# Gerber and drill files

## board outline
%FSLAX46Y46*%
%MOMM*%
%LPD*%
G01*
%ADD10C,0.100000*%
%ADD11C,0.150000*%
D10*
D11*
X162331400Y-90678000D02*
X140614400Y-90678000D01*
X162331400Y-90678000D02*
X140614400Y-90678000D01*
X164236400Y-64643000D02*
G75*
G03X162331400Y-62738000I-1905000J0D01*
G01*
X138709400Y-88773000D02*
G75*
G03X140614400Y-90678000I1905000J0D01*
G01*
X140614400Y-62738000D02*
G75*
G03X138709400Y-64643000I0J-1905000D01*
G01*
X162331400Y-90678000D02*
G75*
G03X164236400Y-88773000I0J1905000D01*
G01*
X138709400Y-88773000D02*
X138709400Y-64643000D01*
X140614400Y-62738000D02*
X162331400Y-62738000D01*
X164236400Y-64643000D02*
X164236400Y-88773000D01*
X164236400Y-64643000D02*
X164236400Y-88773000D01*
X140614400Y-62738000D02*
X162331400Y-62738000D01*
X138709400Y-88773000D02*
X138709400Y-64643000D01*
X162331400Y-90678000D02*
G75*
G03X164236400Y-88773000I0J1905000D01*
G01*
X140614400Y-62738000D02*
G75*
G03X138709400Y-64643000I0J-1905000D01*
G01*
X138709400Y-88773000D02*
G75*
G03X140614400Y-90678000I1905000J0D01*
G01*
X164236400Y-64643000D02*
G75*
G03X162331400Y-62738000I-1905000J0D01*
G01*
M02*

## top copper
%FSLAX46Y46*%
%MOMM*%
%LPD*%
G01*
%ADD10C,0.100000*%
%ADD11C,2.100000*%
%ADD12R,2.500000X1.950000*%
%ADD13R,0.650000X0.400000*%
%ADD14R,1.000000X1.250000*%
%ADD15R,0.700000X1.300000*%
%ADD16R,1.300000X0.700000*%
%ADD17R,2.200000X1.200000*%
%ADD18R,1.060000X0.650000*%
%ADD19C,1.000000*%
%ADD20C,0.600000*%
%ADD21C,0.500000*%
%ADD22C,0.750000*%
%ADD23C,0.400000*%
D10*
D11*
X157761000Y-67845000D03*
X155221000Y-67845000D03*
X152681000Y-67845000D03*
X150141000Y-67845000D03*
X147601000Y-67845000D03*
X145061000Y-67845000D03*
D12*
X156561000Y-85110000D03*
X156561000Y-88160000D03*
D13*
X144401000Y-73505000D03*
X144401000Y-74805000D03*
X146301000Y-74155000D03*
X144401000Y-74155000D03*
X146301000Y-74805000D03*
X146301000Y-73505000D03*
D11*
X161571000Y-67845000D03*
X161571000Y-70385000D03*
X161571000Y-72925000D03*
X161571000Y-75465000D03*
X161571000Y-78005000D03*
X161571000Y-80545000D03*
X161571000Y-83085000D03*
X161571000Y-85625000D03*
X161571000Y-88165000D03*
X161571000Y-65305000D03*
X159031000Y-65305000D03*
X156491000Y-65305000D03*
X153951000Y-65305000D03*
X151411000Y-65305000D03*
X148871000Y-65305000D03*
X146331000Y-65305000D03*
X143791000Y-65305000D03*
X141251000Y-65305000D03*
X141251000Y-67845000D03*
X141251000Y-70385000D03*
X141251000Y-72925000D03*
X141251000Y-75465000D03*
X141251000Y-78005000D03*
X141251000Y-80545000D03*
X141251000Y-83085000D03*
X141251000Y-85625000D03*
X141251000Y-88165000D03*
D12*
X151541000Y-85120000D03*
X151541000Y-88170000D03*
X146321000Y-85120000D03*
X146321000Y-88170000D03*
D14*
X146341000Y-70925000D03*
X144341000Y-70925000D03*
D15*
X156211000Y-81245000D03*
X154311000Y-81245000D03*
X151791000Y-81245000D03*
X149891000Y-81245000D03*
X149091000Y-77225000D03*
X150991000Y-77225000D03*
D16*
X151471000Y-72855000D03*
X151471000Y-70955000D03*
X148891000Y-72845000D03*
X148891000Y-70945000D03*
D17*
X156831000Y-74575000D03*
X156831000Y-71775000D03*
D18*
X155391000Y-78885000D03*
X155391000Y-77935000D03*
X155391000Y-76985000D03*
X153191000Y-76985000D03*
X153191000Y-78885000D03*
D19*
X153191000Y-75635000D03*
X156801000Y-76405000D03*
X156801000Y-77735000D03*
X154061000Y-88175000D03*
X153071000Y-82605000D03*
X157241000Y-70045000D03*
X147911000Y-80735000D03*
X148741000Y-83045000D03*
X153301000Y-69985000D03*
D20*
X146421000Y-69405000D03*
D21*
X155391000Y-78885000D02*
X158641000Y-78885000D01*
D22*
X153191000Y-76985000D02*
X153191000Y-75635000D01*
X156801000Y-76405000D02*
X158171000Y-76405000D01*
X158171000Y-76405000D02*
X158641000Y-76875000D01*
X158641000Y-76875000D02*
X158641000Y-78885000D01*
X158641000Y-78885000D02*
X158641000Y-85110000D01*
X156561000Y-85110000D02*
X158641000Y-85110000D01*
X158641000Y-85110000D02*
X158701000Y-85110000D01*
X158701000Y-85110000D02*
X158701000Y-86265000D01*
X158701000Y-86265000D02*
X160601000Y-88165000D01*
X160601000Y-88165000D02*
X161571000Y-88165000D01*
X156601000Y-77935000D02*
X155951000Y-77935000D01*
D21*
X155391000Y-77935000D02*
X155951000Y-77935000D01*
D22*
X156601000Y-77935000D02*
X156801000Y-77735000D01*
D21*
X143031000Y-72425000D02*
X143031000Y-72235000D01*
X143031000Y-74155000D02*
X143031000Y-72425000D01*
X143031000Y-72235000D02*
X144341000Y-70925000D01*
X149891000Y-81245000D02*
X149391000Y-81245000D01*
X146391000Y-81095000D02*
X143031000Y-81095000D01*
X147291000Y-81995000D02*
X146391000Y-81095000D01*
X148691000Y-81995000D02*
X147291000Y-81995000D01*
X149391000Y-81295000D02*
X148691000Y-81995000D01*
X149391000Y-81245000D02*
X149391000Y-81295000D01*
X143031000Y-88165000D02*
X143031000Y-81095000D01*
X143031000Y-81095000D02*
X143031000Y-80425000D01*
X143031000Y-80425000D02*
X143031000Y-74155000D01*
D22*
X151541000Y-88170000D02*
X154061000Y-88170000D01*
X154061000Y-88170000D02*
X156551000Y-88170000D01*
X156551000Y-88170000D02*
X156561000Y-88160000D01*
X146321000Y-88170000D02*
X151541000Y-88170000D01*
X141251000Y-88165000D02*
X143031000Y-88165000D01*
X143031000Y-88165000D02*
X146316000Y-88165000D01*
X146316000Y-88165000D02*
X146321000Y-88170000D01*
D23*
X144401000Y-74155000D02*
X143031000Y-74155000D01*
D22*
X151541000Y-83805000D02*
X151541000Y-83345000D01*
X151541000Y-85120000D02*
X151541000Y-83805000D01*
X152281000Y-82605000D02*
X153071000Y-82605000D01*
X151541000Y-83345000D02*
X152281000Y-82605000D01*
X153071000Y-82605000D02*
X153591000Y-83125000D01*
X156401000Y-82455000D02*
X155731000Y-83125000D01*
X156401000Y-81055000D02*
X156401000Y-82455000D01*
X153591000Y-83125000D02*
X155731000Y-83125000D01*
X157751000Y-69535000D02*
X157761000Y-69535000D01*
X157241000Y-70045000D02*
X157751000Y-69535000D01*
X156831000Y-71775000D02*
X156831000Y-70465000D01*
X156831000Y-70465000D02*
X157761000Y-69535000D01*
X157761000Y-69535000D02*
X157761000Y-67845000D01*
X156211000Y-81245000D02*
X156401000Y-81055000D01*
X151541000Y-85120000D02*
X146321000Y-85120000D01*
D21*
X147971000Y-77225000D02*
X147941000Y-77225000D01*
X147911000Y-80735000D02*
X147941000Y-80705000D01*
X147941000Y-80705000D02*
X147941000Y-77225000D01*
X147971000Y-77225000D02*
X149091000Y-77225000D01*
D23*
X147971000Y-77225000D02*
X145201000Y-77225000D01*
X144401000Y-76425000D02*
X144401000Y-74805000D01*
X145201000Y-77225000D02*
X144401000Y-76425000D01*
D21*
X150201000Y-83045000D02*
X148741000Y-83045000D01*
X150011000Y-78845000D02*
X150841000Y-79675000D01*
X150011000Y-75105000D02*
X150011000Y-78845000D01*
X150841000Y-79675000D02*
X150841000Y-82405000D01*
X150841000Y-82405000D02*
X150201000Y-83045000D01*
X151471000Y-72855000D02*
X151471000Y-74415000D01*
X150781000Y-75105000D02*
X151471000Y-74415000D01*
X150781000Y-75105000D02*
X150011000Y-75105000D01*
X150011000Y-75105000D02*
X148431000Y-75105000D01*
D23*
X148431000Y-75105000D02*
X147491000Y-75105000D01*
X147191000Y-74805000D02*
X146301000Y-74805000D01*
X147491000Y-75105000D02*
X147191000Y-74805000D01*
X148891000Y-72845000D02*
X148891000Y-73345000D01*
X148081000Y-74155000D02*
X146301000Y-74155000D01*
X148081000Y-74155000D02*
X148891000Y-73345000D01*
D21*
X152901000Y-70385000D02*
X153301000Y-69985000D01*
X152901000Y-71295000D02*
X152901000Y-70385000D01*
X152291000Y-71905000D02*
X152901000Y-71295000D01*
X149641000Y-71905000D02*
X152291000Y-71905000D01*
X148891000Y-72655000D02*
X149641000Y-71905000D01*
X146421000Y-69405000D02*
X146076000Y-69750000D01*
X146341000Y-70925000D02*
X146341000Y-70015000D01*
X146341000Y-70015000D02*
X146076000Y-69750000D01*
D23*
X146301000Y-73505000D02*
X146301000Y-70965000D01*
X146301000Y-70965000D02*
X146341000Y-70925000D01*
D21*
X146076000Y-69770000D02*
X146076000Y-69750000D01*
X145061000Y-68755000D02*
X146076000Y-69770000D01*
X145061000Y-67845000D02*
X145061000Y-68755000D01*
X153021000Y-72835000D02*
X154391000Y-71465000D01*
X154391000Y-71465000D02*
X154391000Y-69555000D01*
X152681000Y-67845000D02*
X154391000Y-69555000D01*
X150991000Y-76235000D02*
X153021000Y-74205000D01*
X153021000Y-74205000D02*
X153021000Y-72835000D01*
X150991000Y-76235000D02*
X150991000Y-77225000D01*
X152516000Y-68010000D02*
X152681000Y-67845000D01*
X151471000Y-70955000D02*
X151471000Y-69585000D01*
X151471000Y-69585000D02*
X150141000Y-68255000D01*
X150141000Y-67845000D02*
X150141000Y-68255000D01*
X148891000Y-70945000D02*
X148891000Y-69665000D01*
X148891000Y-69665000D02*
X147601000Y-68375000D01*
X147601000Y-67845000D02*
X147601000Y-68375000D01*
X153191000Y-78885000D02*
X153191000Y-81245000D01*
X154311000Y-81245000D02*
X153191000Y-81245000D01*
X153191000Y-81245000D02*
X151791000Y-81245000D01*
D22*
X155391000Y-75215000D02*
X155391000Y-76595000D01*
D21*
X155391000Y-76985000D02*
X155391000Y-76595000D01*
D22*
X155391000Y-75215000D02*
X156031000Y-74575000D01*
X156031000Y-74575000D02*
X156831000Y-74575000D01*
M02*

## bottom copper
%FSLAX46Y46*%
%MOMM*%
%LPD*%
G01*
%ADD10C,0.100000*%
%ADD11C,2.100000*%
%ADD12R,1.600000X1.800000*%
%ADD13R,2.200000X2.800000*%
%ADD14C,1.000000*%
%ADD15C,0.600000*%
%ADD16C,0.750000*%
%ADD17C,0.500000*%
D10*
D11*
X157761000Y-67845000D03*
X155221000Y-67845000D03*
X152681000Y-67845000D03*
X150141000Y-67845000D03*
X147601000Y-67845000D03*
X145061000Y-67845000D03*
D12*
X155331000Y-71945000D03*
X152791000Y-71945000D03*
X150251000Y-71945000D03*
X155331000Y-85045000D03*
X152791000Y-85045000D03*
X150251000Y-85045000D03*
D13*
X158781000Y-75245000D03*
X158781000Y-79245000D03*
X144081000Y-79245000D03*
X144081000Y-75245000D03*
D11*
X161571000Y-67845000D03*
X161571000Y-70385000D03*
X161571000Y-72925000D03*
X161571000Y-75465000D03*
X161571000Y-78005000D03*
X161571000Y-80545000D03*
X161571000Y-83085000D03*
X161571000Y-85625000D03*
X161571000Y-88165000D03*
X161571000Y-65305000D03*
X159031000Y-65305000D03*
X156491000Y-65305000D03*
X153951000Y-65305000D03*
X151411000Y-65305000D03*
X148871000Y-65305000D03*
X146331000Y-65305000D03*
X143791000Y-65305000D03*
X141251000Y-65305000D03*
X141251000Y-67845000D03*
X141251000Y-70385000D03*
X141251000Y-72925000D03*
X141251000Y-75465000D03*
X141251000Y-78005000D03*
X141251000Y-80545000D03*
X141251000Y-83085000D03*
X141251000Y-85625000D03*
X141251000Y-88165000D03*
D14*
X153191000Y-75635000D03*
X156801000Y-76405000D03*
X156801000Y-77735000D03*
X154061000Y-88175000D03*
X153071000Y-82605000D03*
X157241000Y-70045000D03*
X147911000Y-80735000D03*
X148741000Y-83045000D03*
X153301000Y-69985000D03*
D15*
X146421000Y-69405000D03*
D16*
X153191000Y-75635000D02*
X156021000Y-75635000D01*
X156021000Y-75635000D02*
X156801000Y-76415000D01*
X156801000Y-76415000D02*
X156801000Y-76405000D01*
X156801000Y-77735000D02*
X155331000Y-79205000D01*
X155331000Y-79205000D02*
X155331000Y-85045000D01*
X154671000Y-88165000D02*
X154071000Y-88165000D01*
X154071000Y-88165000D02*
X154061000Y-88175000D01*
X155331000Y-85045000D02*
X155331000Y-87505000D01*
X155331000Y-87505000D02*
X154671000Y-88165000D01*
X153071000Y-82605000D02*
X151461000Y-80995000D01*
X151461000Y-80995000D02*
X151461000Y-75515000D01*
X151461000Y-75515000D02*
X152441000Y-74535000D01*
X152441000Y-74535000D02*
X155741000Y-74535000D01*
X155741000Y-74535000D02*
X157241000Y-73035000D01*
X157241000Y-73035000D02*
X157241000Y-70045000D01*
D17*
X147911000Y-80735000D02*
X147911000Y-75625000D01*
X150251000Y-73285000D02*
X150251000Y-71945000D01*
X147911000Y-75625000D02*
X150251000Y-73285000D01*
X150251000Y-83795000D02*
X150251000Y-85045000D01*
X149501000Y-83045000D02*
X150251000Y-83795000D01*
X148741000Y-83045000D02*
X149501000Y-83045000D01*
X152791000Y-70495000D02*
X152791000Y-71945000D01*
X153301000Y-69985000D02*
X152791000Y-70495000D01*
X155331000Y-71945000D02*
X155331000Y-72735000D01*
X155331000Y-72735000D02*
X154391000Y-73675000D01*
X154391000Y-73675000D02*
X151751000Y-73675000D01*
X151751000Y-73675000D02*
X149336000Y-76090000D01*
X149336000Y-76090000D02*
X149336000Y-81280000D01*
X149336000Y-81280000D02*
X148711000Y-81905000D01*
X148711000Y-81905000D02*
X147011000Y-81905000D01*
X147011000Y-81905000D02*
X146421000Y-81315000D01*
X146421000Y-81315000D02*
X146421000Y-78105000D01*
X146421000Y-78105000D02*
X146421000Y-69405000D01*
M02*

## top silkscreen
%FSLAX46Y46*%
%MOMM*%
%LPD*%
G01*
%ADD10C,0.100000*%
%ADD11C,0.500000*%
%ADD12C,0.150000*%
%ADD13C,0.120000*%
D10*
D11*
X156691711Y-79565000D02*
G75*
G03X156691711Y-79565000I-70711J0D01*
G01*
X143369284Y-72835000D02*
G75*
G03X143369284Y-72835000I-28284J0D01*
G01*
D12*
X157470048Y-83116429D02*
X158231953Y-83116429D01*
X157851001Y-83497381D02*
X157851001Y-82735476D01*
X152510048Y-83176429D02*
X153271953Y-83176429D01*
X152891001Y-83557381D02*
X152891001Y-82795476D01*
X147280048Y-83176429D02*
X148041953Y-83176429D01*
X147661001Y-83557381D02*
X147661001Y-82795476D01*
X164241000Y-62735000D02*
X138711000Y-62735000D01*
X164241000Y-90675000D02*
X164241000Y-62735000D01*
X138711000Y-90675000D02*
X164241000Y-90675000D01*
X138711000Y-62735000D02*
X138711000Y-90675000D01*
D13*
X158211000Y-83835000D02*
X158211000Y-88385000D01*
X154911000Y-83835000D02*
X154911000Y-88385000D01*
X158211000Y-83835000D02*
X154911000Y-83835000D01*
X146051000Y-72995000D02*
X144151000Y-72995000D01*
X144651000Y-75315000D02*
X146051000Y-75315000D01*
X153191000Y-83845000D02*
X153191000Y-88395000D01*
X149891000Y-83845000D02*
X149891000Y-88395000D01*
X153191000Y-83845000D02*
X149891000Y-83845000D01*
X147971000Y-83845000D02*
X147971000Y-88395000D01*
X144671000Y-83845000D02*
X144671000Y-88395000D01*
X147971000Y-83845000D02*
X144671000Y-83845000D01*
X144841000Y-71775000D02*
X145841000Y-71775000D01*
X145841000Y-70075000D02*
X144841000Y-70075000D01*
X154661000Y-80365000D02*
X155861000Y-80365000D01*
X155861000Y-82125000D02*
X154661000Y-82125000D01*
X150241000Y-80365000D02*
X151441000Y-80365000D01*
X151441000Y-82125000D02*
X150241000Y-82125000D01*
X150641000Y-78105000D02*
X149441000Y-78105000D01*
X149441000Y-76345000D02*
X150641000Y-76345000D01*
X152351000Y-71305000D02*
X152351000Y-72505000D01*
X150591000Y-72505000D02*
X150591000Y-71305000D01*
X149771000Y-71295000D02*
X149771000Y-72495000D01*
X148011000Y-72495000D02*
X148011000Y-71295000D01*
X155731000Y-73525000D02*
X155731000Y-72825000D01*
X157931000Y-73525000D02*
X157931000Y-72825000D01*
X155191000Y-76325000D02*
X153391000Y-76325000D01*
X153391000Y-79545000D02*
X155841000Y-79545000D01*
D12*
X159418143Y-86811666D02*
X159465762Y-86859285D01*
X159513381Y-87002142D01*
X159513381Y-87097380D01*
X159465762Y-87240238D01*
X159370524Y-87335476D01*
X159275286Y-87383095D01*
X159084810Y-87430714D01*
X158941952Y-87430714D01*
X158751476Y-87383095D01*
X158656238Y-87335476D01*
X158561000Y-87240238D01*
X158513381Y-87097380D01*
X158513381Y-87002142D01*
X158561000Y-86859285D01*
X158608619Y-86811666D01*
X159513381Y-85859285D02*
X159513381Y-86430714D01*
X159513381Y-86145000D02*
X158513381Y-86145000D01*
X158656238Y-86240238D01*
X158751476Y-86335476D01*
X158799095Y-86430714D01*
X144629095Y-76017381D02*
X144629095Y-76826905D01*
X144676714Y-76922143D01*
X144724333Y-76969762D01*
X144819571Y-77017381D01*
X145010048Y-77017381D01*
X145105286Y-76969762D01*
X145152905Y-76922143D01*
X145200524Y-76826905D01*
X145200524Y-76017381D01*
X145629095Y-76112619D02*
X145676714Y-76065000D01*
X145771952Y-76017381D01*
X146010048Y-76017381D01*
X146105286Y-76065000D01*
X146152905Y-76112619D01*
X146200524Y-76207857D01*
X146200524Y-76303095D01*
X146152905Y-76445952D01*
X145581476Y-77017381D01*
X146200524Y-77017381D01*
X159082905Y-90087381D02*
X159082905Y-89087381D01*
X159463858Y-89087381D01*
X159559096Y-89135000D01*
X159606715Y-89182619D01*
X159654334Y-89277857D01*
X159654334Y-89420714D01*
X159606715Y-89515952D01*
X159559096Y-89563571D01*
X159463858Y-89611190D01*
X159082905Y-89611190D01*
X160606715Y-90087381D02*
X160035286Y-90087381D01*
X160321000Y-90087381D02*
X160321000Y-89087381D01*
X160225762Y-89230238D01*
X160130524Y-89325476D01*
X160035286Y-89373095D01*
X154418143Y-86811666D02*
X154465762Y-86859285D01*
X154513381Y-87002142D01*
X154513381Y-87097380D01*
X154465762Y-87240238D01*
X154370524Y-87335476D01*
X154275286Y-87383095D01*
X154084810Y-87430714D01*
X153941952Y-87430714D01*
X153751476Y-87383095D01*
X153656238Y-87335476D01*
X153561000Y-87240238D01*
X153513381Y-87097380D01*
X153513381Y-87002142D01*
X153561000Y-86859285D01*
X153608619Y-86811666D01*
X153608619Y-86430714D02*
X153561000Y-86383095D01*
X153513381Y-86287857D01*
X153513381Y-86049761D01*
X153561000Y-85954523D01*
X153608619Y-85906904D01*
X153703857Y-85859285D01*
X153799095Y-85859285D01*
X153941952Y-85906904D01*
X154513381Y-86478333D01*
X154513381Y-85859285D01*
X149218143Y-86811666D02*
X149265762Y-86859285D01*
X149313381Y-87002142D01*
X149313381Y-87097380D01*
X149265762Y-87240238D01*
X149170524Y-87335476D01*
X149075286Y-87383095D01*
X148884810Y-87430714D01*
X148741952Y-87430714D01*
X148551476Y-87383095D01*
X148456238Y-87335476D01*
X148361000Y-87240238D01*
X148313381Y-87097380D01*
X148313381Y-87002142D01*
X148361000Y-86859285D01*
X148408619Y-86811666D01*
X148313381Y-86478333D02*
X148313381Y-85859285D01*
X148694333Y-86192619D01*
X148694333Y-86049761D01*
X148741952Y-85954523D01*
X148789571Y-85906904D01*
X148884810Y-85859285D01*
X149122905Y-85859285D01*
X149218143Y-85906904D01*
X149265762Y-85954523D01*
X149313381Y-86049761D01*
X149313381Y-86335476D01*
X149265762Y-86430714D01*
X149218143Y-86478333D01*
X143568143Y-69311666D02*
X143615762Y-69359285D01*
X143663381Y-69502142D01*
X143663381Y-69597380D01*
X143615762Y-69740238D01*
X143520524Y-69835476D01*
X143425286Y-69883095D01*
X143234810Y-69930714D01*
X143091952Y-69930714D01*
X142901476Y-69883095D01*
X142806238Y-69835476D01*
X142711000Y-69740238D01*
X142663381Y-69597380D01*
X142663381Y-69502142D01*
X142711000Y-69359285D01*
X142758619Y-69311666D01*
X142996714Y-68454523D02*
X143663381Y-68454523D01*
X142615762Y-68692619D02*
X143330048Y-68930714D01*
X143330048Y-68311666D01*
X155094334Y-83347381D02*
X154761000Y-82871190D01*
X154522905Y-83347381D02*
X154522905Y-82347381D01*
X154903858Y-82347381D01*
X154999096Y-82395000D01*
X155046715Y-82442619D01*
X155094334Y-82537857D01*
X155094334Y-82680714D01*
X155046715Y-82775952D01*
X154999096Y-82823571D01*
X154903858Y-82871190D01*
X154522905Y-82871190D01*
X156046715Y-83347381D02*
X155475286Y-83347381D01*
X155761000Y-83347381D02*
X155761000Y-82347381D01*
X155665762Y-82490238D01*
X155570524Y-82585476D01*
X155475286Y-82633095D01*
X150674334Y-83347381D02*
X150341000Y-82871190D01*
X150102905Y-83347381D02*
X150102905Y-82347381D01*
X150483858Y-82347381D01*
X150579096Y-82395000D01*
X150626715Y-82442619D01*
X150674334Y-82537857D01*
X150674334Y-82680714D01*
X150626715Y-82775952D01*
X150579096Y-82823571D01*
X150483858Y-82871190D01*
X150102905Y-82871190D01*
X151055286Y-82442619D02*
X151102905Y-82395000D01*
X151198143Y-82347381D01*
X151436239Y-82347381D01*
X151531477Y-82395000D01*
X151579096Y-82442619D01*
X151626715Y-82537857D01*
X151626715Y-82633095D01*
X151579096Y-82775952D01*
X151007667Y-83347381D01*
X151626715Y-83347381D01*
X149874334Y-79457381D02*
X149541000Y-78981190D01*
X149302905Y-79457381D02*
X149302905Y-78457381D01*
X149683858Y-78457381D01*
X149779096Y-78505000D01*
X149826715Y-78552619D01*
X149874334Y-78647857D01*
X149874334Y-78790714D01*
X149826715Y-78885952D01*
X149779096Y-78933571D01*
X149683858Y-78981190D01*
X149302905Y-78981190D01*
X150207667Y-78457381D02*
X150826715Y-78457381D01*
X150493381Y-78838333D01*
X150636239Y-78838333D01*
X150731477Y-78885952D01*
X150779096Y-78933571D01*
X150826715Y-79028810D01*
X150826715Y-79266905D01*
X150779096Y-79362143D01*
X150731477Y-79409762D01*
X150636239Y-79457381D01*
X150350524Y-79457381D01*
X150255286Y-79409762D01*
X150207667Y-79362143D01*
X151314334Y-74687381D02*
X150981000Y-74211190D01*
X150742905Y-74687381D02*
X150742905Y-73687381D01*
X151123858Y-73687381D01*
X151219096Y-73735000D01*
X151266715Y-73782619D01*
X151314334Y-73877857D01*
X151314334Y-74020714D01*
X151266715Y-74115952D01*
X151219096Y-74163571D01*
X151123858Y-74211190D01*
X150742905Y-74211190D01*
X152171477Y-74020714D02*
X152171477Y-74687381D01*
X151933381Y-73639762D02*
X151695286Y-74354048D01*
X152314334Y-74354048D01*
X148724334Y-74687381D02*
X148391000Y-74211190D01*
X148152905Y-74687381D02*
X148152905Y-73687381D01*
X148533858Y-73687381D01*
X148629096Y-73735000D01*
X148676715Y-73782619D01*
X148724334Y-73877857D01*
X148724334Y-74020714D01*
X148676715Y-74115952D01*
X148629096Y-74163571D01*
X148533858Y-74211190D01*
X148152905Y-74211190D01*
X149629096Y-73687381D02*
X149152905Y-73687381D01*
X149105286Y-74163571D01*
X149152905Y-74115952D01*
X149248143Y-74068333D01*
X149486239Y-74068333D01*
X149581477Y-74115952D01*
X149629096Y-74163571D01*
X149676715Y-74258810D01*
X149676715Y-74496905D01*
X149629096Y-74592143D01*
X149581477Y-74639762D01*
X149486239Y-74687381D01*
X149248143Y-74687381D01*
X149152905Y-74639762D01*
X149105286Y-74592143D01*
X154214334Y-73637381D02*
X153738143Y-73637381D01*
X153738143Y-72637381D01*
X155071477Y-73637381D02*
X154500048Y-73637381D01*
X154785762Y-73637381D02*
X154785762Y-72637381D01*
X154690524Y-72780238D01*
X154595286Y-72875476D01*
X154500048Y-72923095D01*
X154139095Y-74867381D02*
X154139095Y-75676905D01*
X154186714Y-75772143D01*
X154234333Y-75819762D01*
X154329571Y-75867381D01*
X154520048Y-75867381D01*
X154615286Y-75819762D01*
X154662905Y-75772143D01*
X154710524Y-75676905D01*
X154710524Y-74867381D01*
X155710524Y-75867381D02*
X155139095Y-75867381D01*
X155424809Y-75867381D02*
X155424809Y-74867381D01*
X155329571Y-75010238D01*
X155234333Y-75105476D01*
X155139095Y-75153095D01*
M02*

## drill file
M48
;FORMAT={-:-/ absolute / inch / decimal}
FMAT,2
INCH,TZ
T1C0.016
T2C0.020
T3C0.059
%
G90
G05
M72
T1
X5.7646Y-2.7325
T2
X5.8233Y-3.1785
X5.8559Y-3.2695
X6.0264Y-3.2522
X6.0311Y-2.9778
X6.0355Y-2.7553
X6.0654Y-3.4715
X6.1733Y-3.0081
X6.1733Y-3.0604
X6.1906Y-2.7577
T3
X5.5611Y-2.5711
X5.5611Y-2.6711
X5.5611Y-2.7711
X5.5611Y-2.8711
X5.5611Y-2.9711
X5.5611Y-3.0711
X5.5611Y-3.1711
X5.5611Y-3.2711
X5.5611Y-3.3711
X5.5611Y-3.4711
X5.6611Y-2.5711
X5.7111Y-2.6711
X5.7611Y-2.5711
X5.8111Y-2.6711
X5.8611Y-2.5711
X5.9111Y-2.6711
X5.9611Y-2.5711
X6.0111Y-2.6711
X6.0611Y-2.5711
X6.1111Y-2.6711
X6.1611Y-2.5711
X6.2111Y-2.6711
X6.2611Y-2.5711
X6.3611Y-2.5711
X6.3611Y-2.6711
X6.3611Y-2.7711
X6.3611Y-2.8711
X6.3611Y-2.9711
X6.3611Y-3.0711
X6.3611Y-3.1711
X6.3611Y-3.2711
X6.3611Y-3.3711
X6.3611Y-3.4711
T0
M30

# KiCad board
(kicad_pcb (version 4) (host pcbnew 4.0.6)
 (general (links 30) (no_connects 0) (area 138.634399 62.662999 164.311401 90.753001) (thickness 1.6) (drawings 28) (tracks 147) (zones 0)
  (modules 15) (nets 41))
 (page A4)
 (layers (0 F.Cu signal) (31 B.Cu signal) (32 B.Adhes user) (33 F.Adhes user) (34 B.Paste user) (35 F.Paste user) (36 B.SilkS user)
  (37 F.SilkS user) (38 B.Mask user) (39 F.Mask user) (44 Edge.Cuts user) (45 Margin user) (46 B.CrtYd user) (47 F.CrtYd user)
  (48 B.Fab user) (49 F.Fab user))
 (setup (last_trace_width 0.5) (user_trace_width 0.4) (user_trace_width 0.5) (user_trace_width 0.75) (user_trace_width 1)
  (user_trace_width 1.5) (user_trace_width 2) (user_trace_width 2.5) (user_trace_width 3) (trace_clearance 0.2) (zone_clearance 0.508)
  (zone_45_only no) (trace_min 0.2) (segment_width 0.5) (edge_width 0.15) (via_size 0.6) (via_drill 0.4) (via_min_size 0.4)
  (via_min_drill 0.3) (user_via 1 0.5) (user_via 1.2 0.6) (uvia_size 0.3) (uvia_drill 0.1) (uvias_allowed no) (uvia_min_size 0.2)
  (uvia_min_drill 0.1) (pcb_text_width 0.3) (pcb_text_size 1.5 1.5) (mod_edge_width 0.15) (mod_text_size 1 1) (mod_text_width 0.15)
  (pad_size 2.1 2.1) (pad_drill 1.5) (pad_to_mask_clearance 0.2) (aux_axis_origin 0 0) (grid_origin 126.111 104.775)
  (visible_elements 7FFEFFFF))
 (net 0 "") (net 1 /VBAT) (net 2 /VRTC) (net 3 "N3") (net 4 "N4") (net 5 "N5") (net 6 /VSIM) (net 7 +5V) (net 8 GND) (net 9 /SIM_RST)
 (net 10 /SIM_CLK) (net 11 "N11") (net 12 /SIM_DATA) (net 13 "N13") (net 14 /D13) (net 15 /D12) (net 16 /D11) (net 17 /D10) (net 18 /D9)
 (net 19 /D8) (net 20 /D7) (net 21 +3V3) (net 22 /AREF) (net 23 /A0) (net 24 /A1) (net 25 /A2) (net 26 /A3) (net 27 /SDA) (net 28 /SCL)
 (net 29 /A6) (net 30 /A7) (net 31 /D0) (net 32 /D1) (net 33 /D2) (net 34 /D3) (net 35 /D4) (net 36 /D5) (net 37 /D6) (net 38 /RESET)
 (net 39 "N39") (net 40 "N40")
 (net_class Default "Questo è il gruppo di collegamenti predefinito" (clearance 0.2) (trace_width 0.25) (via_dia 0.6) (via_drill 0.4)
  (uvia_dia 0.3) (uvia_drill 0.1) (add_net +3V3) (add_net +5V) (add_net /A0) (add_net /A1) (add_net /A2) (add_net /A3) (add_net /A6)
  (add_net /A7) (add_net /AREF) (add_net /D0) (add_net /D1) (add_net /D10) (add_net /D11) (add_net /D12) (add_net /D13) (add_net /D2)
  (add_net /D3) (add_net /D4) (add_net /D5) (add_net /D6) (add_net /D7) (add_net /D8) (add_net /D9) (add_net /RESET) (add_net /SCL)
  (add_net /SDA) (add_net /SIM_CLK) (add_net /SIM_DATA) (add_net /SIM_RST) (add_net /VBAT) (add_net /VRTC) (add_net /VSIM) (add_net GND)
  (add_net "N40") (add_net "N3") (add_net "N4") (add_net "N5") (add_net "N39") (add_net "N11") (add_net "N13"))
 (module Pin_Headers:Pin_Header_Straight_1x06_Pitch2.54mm (layer B.Cu) (at 157.761 67.845 90)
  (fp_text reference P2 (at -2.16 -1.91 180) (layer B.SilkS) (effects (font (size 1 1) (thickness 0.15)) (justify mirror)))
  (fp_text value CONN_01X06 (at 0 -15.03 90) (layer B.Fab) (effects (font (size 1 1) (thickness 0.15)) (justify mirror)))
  (pad 1 thru_hole circle (at 0 0 90) (size 2.1 2.1) (drill 1.5) (layers *.Cu *.Mask) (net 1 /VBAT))
  (pad 2 thru_hole circle (at 0 -2.54 90) (size 2.1 2.1) (drill 1.5) (layers *.Cu *.Mask) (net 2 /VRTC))
  (pad 3 thru_hole circle (at 0 -5.08 90) (size 2.1 2.1) (drill 1.5) (layers *.Cu *.Mask) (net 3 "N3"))
  (pad 4 thru_hole circle (at 0 -7.62 90) (size 2.1 2.1) (drill 1.5) (layers *.Cu *.Mask) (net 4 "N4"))
  (pad 5 thru_hole circle (at 0 -10.16 90) (size 2.1 2.1) (drill 1.5) (layers *.Cu *.Mask) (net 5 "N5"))
  (pad 6 thru_hole circle (at 0 -12.7 90) (size 2.1 2.1) (drill 1.5) (layers *.Cu *.Mask) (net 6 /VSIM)))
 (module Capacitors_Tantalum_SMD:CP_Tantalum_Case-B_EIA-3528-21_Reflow (layer F.Cu) (at 156.561 86.635 270)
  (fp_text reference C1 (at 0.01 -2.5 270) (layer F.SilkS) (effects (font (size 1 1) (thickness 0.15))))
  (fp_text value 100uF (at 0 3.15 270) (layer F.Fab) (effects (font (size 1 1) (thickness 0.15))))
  (fp_line (start -2.8 -1.65) (end 1.75 -1.65) (layer F.SilkS) (width 0.12))
  (fp_line (start -2.8 1.65) (end 1.75 1.65) (layer F.SilkS) (width 0.12))
  (fp_line (start -2.8 -1.65) (end -2.8 1.65) (layer F.SilkS) (width 0.12))
  (pad 1 smd rect (at -1.525 0 270) (size 1.95 2.5) (layers F.Cu F.Paste F.Mask) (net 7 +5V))
  (pad 2 smd rect (at 1.525 0 270) (size 1.95 2.5) (layers F.Cu F.Paste F.Mask) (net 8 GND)))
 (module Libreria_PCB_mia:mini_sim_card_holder (layer B.Cu) (at 151.431 77.245 180)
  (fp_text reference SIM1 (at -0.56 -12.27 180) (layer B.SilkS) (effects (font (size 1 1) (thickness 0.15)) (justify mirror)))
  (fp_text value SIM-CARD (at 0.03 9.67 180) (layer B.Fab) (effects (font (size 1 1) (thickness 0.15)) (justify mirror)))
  (pad 1 smd rect (at -3.9 5.3 180) (size 1.6 1.8) (layers B.Cu B.Paste B.Mask) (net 6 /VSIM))
  (pad 2 smd rect (at -1.36 5.3 180) (size 1.6 1.8) (layers B.Cu B.Paste B.Mask) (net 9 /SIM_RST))
  (pad 3 smd rect (at 1.18 5.3 180) (size 1.6 1.8) (layers B.Cu B.Paste B.Mask) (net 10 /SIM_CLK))
  (pad 4 smd rect (at -3.9 -7.8 180) (size 1.6 1.8) (layers B.Cu B.Paste B.Mask) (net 8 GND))
  (pad 5 smd rect (at -1.36 -7.8 180) (size 1.6 1.8) (layers B.Cu B.Paste B.Mask) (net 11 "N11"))
  (pad 6 smd rect (at 1.18 -7.8 180) (size 1.6 1.8) (layers B.Cu B.Paste B.Mask) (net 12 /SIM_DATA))
  (pad "" smd rect (at -7.35 2 180) (size 2.2 2.8) (layers B.Cu B.Paste B.Mask))
  (pad "" smd rect (at -7.35 -2 180) (size 2.2 2.8) (layers B.Cu B.Paste B.Mask))
  (pad "" smd rect (at 7.35 -2 180) (size 2.2 2.8) (layers B.Cu B.Paste B.Mask))
  (pad "" smd rect (at 7.35 2 180) (size 2.2 2.8) (layers B.Cu B.Paste B.Mask)))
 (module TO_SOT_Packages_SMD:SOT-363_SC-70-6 (layer F.Cu) (at 145.351 74.155)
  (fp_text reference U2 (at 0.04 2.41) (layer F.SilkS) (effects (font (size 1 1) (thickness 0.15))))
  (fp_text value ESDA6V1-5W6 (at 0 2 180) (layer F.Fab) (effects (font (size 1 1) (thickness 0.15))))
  (fp_line (start 0.7 -1.16) (end -1.2 -1.16) (layer F.SilkS) (width 0.12))
  (fp_line (start -0.7 1.16) (end 0.7 1.16) (layer F.SilkS) (width 0.12))
  (pad 1 smd rect (at -0.95 -0.65) (size 0.65 0.4) (layers F.Cu F.Paste F.Mask) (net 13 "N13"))
  (pad 3 smd rect (at -0.95 0.65) (size 0.65 0.4) (layers F.Cu F.Paste F.Mask) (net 10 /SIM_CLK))
  (pad 5 smd rect (at 0.95 0) (size 0.65 0.4) (layers F.Cu F.Paste F.Mask) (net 9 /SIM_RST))
  (pad 2 smd rect (at -0.95 0) (size 0.65 0.4) (layers F.Cu F.Paste F.Mask) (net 8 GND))
  (pad 4 smd rect (at 0.95 0.65) (size 0.65 0.4) (layers F.Cu F.Paste F.Mask) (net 12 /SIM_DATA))
  (pad 6 smd rect (at 0.95 -0.65) (size 0.65 0.4) (layers F.Cu F.Paste F.Mask) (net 6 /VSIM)))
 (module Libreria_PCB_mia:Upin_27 (layer B.Cu) (at 161.571 88.165 180)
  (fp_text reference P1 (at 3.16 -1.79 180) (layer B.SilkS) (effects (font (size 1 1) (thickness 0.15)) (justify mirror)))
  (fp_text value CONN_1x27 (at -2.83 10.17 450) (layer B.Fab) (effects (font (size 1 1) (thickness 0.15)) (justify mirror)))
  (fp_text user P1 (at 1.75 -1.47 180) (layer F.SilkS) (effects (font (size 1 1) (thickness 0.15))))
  (pad 9 thru_hole circle (at 0 20.32 180) (size 2.1 2.1) (drill 1.5) (layers *.Cu *.Mask) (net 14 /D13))
  (pad 8 thru_hole circle (at 0 17.78 180) (size 2.1 2.1) (drill 1.5) (layers *.Cu *.Mask) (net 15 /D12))
  (pad 7 thru_hole circle (at 0 15.24 180) (size 2.1 2.1) (drill 1.5) (layers *.Cu *.Mask) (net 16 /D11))
  (pad 6 thru_hole circle (at 0 12.7 180) (size 2.1 2.1) (drill 1.5) (layers *.Cu *.Mask) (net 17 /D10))
  (pad 5 thru_hole circle (at 0 10.16 180) (size 2.1 2.1) (drill 1.5) (layers *.Cu *.Mask) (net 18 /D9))
  (pad 4 thru_hole circle (at 0 7.62 180) (size 2.1 2.1) (drill 1.5) (layers *.Cu *.Mask) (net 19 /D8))
  (pad 3 thru_hole circle (at 0 5.08 180) (size 2.1 2.1) (drill 1.5) (layers *.Cu *.Mask) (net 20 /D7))
  (pad 2 thru_hole circle (at 0 2.54 180) (size 2.1 2.1) (drill 1.5) (layers *.Cu *.Mask) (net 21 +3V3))
  (pad 1 thru_hole circle (at 0 0 180) (size 2.1 2.1) (drill 1.5) (layers *.Cu *.Mask) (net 7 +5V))
  (pad 10 thru_hole circle (at 0 22.86 180) (size 2.1 2.1) (drill 1.5) (layers *.Cu *.Mask) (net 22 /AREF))
  (pad 11 thru_hole circle (at 2.54 22.86 180) (size 2.1 2.1) (drill 1.5) (layers *.Cu *.Mask) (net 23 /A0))
  (pad 12 thru_hole circle (at 5.08 22.86 180) (size 2.1 2.1) (drill 1.5) (layers *.Cu *.Mask) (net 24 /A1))
  (pad 13 thru_hole circle (at 7.62 22.86 180) (size 2.1 2.1) (drill 1.5) (layers *.Cu *.Mask) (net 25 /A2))
  (pad 14 thru_hole circle (at 10.16 22.86 180) (size 2.1 2.1) (drill 1.5) (layers *.Cu *.Mask) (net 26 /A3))
  (pad 15 thru_hole circle (at 12.7 22.86 180) (size 2.1 2.1) (drill 1.5) (layers *.Cu *.Mask) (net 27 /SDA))
  (pad 16 thru_hole circle (at 15.24 22.86 180) (size 2.1 2.1) (drill 1.5) (layers *.Cu *.Mask) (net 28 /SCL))
  (pad 17 thru_hole circle (at 17.78 22.86 180) (size 2.1 2.1) (drill 1.5) (layers *.Cu *.Mask) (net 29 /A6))
  (pad 18 thru_hole circle (at 20.32 22.86 180) (size 2.1 2.1) (drill 1.5) (layers *.Cu *.Mask) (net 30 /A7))
  (pad 19 thru_hole circle (at 20.32 20.32 180) (size 2.1 2.1) (drill 1.5) (layers *.Cu *.Mask) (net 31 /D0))
  (pad 20 thru_hole circle (at 20.32 17.78 180) (size 2.1 2.1) (drill 1.5) (layers *.Cu *.Mask) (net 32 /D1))
  (pad 21 thru_hole circle (at 20.32 15.24 180) (size 2.1 2.1) (drill 1.5) (layers *.Cu *.Mask) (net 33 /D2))
  (pad 22 thru_hole circle (at 20.32 12.7 180) (size 2.1 2.1) (drill 1.5) (layers *.Cu *.Mask) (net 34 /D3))
  (pad 23 thru_hole circle (at 20.32 10.16 180) (size 2.1 2.1) (drill 1.5) (layers *.Cu *.Mask) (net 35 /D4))
  (pad 24 thru_hole circle (at 20.32 7.62 180) (size 2.1 2.1) (drill 1.5) (layers *.Cu *.Mask) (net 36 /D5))
  (pad 25 thru_hole circle (at 20.32 5.08 180) (size 2.1 2.1) (drill 1.5) (layers *.Cu *.Mask) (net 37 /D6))
  (pad 26 thru_hole circle (at 20.32 2.54 180) (size 2.1 2.1) (drill 1.5) (layers *.Cu *.Mask) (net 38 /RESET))
  (pad 27 thru_hole circle (at 20.32 0 180) (size 2.1 2.1) (drill 1.5) (layers *.Cu *.Mask) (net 8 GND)))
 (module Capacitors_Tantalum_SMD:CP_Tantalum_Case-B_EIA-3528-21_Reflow (layer F.Cu) (at 151.541 86.645 270)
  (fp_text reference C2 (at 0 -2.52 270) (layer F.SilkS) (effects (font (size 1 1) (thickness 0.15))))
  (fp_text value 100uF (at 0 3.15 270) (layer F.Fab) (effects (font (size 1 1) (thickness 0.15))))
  (fp_line (start -2.8 -1.65) (end 1.75 -1.65) (layer F.SilkS) (width 0.12))
  (fp_line (start -2.8 1.65) (end 1.75 1.65) (layer F.SilkS) (width 0.12))
  (fp_line (start -2.8 -1.65) (end -2.8 1.65) (layer F.SilkS) (width 0.12))
  (pad 1 smd rect (at -1.525 0 270) (size 1.95 2.5) (layers F.Cu F.Paste F.Mask) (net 1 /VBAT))
  (pad 2 smd rect (at 1.525 0 270) (size 1.95 2.5) (layers F.Cu F.Paste F.Mask) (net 8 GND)))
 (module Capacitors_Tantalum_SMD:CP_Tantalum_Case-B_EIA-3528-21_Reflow (layer F.Cu) (at 146.321 86.645 270)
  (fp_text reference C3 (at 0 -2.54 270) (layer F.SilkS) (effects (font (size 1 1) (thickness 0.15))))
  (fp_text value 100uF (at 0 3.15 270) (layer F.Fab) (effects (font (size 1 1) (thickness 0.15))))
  (fp_line (start -2.8 -1.65) (end 1.75 -1.65) (layer F.SilkS) (width 0.12))
  (fp_line (start -2.8 1.65) (end 1.75 1.65) (layer F.SilkS) (width 0.12))
  (fp_line (start -2.8 -1.65) (end -2.8 1.65) (layer F.SilkS) (width 0.12))
  (pad 1 smd rect (at -1.525 0 270) (size 1.95 2.5) (layers F.Cu F.Paste F.Mask) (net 1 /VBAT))
  (pad 2 smd rect (at 1.525 0 270) (size 1.95 2.5) (layers F.Cu F.Paste F.Mask) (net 8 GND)))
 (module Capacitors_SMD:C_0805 (layer F.Cu) (at 145.341 70.925 180)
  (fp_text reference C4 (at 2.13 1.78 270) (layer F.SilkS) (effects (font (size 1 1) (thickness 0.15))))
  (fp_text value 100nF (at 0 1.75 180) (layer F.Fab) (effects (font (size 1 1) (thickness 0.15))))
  (fp_line (start 0.5 -0.85) (end -0.5 -0.85) (layer F.SilkS) (width 0.12))
  (fp_line (start -0.5 0.85) (end 0.5 0.85) (layer F.SilkS) (width 0.12))
  (pad 1 smd rect (at -1 0 180) (size 1 1.25) (layers F.Cu F.Paste F.Mask) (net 6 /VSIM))
  (pad 2 smd rect (at 1 0 180) (size 1 1.25) (layers F.Cu F.Paste F.Mask) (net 8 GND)))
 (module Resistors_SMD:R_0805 (layer F.Cu) (at 155.261 81.245 180)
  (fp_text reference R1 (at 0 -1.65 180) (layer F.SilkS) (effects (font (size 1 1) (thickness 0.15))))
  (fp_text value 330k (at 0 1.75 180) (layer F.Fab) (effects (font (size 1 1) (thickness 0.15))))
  (fp_line (start 0.6 0.88) (end -0.6 0.88) (layer F.SilkS) (width 0.12))
  (fp_line (start -0.6 -0.88) (end 0.6 -0.88) (layer F.SilkS) (width 0.12))
  (pad 1 smd rect (at -0.95 0 180) (size 0.7 1.3) (layers F.Cu F.Paste F.Mask) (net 1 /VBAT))
  (pad 2 smd rect (at 0.95 0 180) (size 0.7 1.3) (layers F.Cu F.Paste F.Mask) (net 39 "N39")))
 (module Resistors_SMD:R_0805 (layer F.Cu) (at 150.841 81.245 180)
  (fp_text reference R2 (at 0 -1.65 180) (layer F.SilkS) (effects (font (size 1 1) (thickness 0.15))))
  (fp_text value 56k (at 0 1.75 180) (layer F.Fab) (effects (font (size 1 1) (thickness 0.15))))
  (fp_line (start 0.6 0.88) (end -0.6 0.88) (layer F.SilkS) (width 0.12))
  (fp_line (start -0.6 -0.88) (end 0.6 -0.88) (layer F.SilkS) (width 0.12))
  (pad 1 smd rect (at -0.95 0 180) (size 0.7 1.3) (layers F.Cu F.Paste F.Mask) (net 39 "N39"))
  (pad 2 smd rect (at 0.95 0 180) (size 0.7 1.3) (layers F.Cu F.Paste F.Mask) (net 8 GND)))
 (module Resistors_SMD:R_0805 (layer F.Cu) (at 150.041 77.225)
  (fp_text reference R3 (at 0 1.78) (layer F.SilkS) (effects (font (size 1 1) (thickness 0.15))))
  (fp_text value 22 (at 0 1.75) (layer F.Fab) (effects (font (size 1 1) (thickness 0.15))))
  (fp_line (start 0.6 0.88) (end -0.6 0.88) (layer F.SilkS) (width 0.12))
  (fp_line (start -0.6 -0.88) (end 0.6 -0.88) (layer F.SilkS) (width 0.12))
  (pad 1 smd rect (at -0.95 0) (size 0.7 1.3) (layers F.Cu F.Paste F.Mask) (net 10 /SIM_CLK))
  (pad 2 smd rect (at 0.95 0) (size 0.7 1.3) (layers F.Cu F.Paste F.Mask) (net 3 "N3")))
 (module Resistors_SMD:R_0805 (layer F.Cu) (at 151.471 71.905 90)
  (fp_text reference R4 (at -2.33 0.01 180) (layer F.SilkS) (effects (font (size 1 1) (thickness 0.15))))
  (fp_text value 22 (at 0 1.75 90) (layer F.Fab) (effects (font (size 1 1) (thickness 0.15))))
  (fp_line (start 0.6 0.88) (end -0.6 0.88) (layer F.SilkS) (width 0.12))
  (fp_line (start -0.6 -0.88) (end 0.6 -0.88) (layer F.SilkS) (width 0.12))
  (pad 1 smd rect (at -0.95 0 90) (size 0.7 1.3) (layers F.Cu F.Paste F.Mask) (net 12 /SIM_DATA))
  (pad 2 smd rect (at 0.95 0 90) (size 0.7 1.3) (layers F.Cu F.Paste F.Mask) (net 4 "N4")))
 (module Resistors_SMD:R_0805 (layer F.Cu) (at 148.891 71.895 90)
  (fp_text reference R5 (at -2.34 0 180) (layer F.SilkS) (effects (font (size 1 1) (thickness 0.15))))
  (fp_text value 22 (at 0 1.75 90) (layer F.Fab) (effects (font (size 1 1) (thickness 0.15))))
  (fp_line (start 0.6 0.88) (end -0.6 0.88) (layer F.SilkS) (width 0.12))
  (fp_line (start -0.6 -0.88) (end 0.6 -0.88) (layer F.SilkS) (width 0.12))
  (pad 1 smd rect (at -0.95 0 90) (size 0.7 1.3) (layers F.Cu F.Paste F.Mask) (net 9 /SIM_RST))
  (pad 2 smd rect (at 0.95 0 90) (size 0.7 1.3) (layers F.Cu F.Paste F.Mask) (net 5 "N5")))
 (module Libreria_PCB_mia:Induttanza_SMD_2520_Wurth (layer F.Cu) (at 156.831 73.175 90)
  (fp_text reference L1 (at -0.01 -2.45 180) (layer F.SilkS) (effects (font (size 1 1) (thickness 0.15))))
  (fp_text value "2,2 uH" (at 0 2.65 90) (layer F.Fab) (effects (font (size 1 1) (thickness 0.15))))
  (fp_line (start -0.35 -1.1) (end 0.35 -1.1) (layer F.SilkS) (width 0.12))
  (fp_line (start -0.35 1.1) (end 0.35 1.1) (layer F.SilkS) (width 0.12))
  (pad 1 smd rect (at -1.4 0 90) (size 1.2 2.2) (layers F.Cu F.Paste F.Mask) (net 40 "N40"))
  (pad 2 smd rect (at 1.4 0 90) (size 1.2 2.2) (layers F.Cu F.Paste F.Mask) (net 1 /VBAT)))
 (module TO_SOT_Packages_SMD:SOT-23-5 (layer F.Cu) (at 154.291 77.935 180)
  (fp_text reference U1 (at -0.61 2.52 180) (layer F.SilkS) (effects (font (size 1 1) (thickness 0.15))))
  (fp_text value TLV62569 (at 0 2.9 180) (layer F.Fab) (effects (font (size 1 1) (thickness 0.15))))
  (fp_line (start -0.9 1.61) (end 0.9 1.61) (layer F.SilkS) (width 0.12))
  (fp_line (start 0.9 -1.61) (end -1.55 -1.61) (layer F.SilkS) (width 0.12))
  (pad 1 smd rect (at -1.1 -0.95 180) (size 1.06 0.65) (layers F.Cu F.Paste F.Mask) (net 7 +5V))
  (pad 2 smd rect (at -1.1 0 180) (size 1.06 0.65) (layers F.Cu F.Paste F.Mask) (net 8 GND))
  (pad 3 smd rect (at -1.1 0.95 180) (size 1.06 0.65) (layers F.Cu F.Paste F.Mask) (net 40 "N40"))
  (pad 4 smd rect (at 1.1 0.95 180) (size 1.06 0.65) (layers F.Cu F.Paste F.Mask) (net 7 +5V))
  (pad 5 smd rect (at 1.1 -0.95 180) (size 1.06 0.65) (layers F.Cu F.Paste F.Mask) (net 39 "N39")))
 (gr_circle (center 156.621 79.565) (end 156.691 79.575) (layer F.SilkS) (width 0.5))
 (gr_circle (center 143.341 72.835) (end 143.321 72.815) (layer F.SilkS) (width 0.5))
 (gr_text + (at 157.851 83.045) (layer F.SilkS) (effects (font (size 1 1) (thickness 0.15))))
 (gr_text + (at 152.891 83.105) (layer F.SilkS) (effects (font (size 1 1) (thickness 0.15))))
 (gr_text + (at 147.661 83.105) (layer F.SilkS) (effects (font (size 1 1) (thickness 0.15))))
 (gr_line (start 164.241 62.735) (end 138.711 62.735) (angle 90) (layer F.SilkS) (width 0.15))
 (gr_line (start 164.241 90.675) (end 164.241 62.735) (angle 90) (layer F.SilkS) (width 0.15))
 (gr_line (start 138.711 90.675) (end 164.241 90.675) (angle 90) (layer F.SilkS) (width 0.15))
 (gr_line (start 138.711 62.735) (end 138.711 90.675) (angle 90) (layer F.SilkS) (width 0.15))
 (gr_line (start 162.3314 90.678) (end 140.6144 90.678) (angle 90) (layer Edge.Cuts) (width 0.15))
 (gr_line (start 162.3314 90.678) (end 140.6144 90.678) (angle 90) (layer Edge.Cuts) (width 0.15))
 (gr_arc (start 162.3314 64.643) (end 162.3314 62.738) (angle 90) (layer Edge.Cuts) (width 0.15))
 (gr_arc (start 140.6144 88.773) (end 140.6144 90.678) (angle 90) (layer Edge.Cuts) (width 0.15))
 (gr_arc (start 140.6144 64.643) (end 138.7094 64.643) (angle 90) (layer Edge.Cuts) (width 0.15))
 (gr_arc (start 162.3314 88.773) (end 164.2364 88.773) (angle 90) (layer Edge.Cuts) (width 0.15))
 (gr_line (start 138.7094 88.773) (end 138.7094 64.643) (angle 90) (layer Edge.Cuts) (width 0.15))
 (gr_line (start 140.6144 62.738) (end 162.3314 62.738) (angle 90) (layer Edge.Cuts) (width 0.15))
 (gr_line (start 164.2364 64.643) (end 164.2364 88.773) (angle 90) (layer Edge.Cuts) (width 0.15))
 (gr_line (start 164.2364 64.643) (end 164.2364 88.773) (angle 90) (layer Edge.Cuts) (width 0.15))
 (gr_line (start 140.6144 62.738) (end 162.3314 62.738) (angle 90) (layer Edge.Cuts) (width 0.15))
 (gr_line (start 138.7094 88.773) (end 138.7094 64.643) (angle 90) (layer Edge.Cuts) (width 0.15))
 (gr_arc (start 162.3314 88.773) (end 164.2364 88.773) (angle 90) (layer Edge.Cuts) (width 0.15))
 (gr_arc (start 140.6144 64.643) (end 138.7094 64.643) (angle 90) (layer Edge.Cuts) (width 0.15))
 (gr_arc (start 140.6144 88.773) (end 140.6144 90.678) (angle 90) (layer Edge.Cuts) (width 0.15))
 (gr_arc (start 162.3314 64.643) (end 162.3314 62.738) (angle 90) (layer Edge.Cuts) (width 0.15))
 (segment (start 155.391 78.885) (end 158.641 78.885) (width 0.5) (layer F.Cu) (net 7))
 (segment (start 153.191 76.985) (end 153.191 75.635) (width 0.75) (layer F.Cu) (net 7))
 (via (at 153.191 75.635) (size 1) (drill 0.5) (layers F.Cu B.Cu) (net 7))
 (segment (start 153.191 75.635) (end 156.021 75.635) (width 0.75) (layer B.Cu) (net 7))
 (segment (start 156.021 75.635) (end 156.801 76.415) (width 0.75) (layer B.Cu) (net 7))
 (segment (start 156.801 76.415) (end 156.801 76.405) (width 0.75) (layer B.Cu) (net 7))
 (via (at 156.801 76.405) (size 1) (drill 0.5) (layers F.Cu B.Cu) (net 7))
 (segment (start 156.801 76.405) (end 158.171 76.405) (width 0.75) (layer F.Cu) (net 7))
 (segment (start 158.171 76.405) (end 158.641 76.875) (width 0.75) (layer F.Cu) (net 7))
 (segment (start 158.641 76.875) (end 158.641 78.885) (width 0.75) (layer F.Cu) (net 7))
 (segment (start 158.641 78.885) (end 158.641 85.11) (width 0.75) (layer F.Cu) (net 7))
 (segment (start 156.561 85.11) (end 158.641 85.11) (width 0.75) (layer F.Cu) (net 7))
 (segment (start 158.641 85.11) (end 158.701 85.11) (width 0.75) (layer F.Cu) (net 7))
 (segment (start 158.701 85.11) (end 158.701 86.265) (width 0.75) (layer F.Cu) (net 7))
 (segment (start 158.701 86.265) (end 160.601 88.165) (width 0.75) (layer F.Cu) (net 7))
 (segment (start 160.601 88.165) (end 161.571 88.165) (width 0.75) (layer F.Cu) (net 7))
 (segment (start 156.601 77.935) (end 155.951 77.935) (width 0.75) (layer F.Cu) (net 8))
 (segment (start 155.391 77.935) (end 155.951 77.935) (width 0.5) (layer F.Cu) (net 8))
 (segment (start 156.601 77.935) (end 156.801 77.735) (width 0.75) (layer F.Cu) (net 8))
 (via (at 156.801 77.735) (size 1) (drill 0.5) (layers F.Cu B.Cu) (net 8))
 (segment (start 156.801 77.735) (end 155.331 79.205) (width 0.75) (layer B.Cu) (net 8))
 (segment (start 155.331 79.205) (end 155.331 85.045) (width 0.75) (layer B.Cu) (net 8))
 (segment (start 143.031 72.425) (end 143.031 72.235) (width 0.5) (layer F.Cu) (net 8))
 (segment (start 143.031 74.155) (end 143.031 72.425) (width 0.5) (layer F.Cu) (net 8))
 (segment (start 143.031 72.235) (end 144.341 70.925) (width 0.5) (layer F.Cu) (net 8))
 (segment (start 149.891 81.245) (end 149.391 81.245) (width 0.5) (layer F.Cu) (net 8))
 (segment (start 146.391 81.095) (end 143.031 81.095) (width 0.5) (layer F.Cu) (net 8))
 (segment (start 147.291 81.995) (end 146.391 81.095) (width 0.5) (layer F.Cu) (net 8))
 (segment (start 148.691 81.995) (end 147.291 81.995) (width 0.5) (layer F.Cu) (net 8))
 (segment (start 149.391 81.295) (end 148.691 81.995) (width 0.5) (layer F.Cu) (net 8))
 (segment (start 149.391 81.245) (end 149.391 81.295) (width 0.5) (layer F.Cu) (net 8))
 (segment (start 154.671 88.165) (end 154.071 88.165) (width 0.75) (layer B.Cu) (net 8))
 (segment (start 154.071 88.165) (end 154.061 88.175) (width 0.75) (layer B.Cu) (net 8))
 (via (at 154.061 88.175) (size 1) (drill 0.5) (layers F.Cu B.Cu) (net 8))
 (segment (start 155.331 85.045) (end 155.331 87.505) (width 0.75) (layer B.Cu) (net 8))
 (segment (start 155.331 87.505) (end 154.671 88.165) (width 0.75) (layer B.Cu) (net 8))
 (segment (start 143.031 88.165) (end 143.031 81.095) (width 0.5) (layer F.Cu) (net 8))
 (segment (start 143.031 81.095) (end 143.031 80.425) (width 0.5) (layer F.Cu) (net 8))
 (segment (start 143.031 80.425) (end 143.031 74.155) (width 0.5) (layer F.Cu) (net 8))
 (segment (start 151.541 88.17) (end 154.061 88.17) (width 0.75) (layer F.Cu) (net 8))
 (segment (start 154.061 88.17) (end 156.551 88.17) (width 0.75) (layer F.Cu) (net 8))
 (segment (start 156.551 88.17) (end 156.561 88.16) (width 0.75) (layer F.Cu) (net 8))
 (segment (start 146.321 88.17) (end 151.541 88.17) (width 0.75) (layer F.Cu) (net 8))
 (segment (start 141.251 88.165) (end 143.031 88.165) (width 0.75) (layer F.Cu) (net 8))
 (segment (start 143.031 88.165) (end 146.316 88.165) (width 0.75) (layer F.Cu) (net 8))
 (segment (start 146.316 88.165) (end 146.321 88.17) (width 0.75) (layer F.Cu) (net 8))
 (segment (start 144.401 74.155) (end 143.031 74.155) (width 0.4) (layer F.Cu) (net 8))
 (segment (start 151.541 83.805) (end 151.541 83.345) (width 0.75) (layer F.Cu) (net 1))
 (segment (start 151.541 85.12) (end 151.541 83.805) (width 0.75) (layer F.Cu) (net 1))
 (segment (start 152.281 82.605) (end 153.071 82.605) (width 0.75) (layer F.Cu) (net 1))
 (segment (start 151.541 83.345) (end 152.281 82.605) (width 0.75) (layer F.Cu) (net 1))
 (segment (start 153.071 82.605) (end 153.591 83.125) (width 0.75) (layer F.Cu) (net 1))
 (segment (start 156.401 82.455) (end 155.731 83.125) (width 0.75) (layer F.Cu) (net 1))
 (segment (start 156.401 81.055) (end 156.401 82.455) (width 0.75) (layer F.Cu) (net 1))
 (segment (start 153.591 83.125) (end 155.731 83.125) (width 0.75) (layer F.Cu) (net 1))
 (segment (start 157.751 69.535) (end 157.761 69.535) (width 0.75) (layer F.Cu) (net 1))
 (via (at 153.071 82.605) (size 1) (drill 0.5) (layers F.Cu B.Cu) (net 1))
 (segment (start 153.071 82.605) (end 151.461 80.995) (width 0.75) (layer B.Cu) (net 1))
 (segment (start 151.461 80.995) (end 151.461 75.515) (width 0.75) (layer B.Cu) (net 1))
 (segment (start 151.461 75.515) (end 152.441 74.535) (width 0.75) (layer B.Cu) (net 1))
 (segment (start 152.441 74.535) (end 155.741 74.535) (width 0.75) (layer B.Cu) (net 1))
 (segment (start 155.741 74.535) (end 157.241 73.035) (width 0.75) (layer B.Cu) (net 1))
 (segment (start 157.241 73.035) (end 157.241 70.045) (width 0.75) (layer B.Cu) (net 1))
 (via (at 157.241 70.045) (size 1) (drill 0.5) (layers F.Cu B.Cu) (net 1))
 (segment (start 157.241 70.045) (end 157.751 69.535) (width 0.75) (layer F.Cu) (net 1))
 (segment (start 156.831 71.775) (end 156.831 70.465) (width 0.75) (layer F.Cu) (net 1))
 (segment (start 156.831 70.465) (end 157.761 69.535) (width 0.75) (layer F.Cu) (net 1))
 (segment (start 157.761 69.535) (end 157.761 67.845) (width 0.75) (layer F.Cu) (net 1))
 (segment (start 156.211 81.245) (end 156.401 81.055) (width 0.75) (layer F.Cu) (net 1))
 (segment (start 151.541 85.12) (end 146.321 85.12) (width 0.75) (layer F.Cu) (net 1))
 (segment (start 147.911 80.735) (end 147.911 75.625) (width 0.5) (layer B.Cu) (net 10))
 (segment (start 147.971 77.225) (end 147.941 77.225) (width 0.5) (layer F.Cu) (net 10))
 (via (at 147.911 80.735) (size 1) (drill 0.5) (layers F.Cu B.Cu) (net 10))
 (segment (start 147.911 80.735) (end 147.941 80.705) (width 0.5) (layer F.Cu) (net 10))
 (segment (start 147.941 80.705) (end 147.941 77.225) (width 0.5) (layer F.Cu) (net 10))
 (segment (start 150.251 73.285) (end 150.251 71.945) (width 0.5) (layer B.Cu) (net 10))
 (segment (start 147.911 75.625) (end 150.251 73.285) (width 0.5) (layer B.Cu) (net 10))
 (segment (start 147.971 77.225) (end 149.091 77.225) (width 0.5) (layer F.Cu) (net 10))
 (segment (start 147.971 77.225) (end 145.201 77.225) (width 0.4) (layer F.Cu) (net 10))
 (segment (start 144.401 76.425) (end 144.401 74.805) (width 0.4) (layer F.Cu) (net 10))
 (segment (start 145.201 77.225) (end 144.401 76.425) (width 0.4) (layer F.Cu) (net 10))
 (segment (start 150.201 83.045) (end 148.741 83.045) (width 0.5) (layer F.Cu) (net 12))
 (segment (start 150.011 78.845) (end 150.841 79.675) (width 0.5) (layer F.Cu) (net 12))
 (segment (start 150.011 75.105) (end 150.011 78.845) (width 0.5) (layer F.Cu) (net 12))
 (segment (start 150.841 79.675) (end 150.841 82.405) (width 0.5) (layer F.Cu) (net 12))
 (segment (start 150.841 82.405) (end 150.201 83.045) (width 0.5) (layer F.Cu) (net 12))
 (segment (start 150.251 83.795) (end 150.251 85.045) (width 0.5) (layer B.Cu) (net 12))
 (segment (start 149.501 83.045) (end 150.251 83.795) (width 0.5) (layer B.Cu) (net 12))
 (segment (start 148.741 83.045) (end 149.501 83.045) (width 0.5) (layer B.Cu) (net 12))
 (via (at 148.741 83.045) (size 1) (drill 0.5) (layers F.Cu B.Cu) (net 12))
 (segment (start 151.471 72.855) (end 151.471 74.415) (width 0.5) (layer F.Cu) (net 12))
 (segment (start 150.781 75.105) (end 151.471 74.415) (width 0.5) (layer F.Cu) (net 12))
 (segment (start 150.781 75.105) (end 150.011 75.105) (width 0.5) (layer F.Cu) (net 12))
 (segment (start 150.011 75.105) (end 148.431 75.105) (width 0.5) (layer F.Cu) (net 12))
 (segment (start 148.431 75.105) (end 147.491 75.105) (width 0.4) (layer F.Cu) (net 12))
 (segment (start 147.191 74.805) (end 146.301 74.805) (width 0.4) (layer F.Cu) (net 12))
 (segment (start 147.491 75.105) (end 147.191 74.805) (width 0.4) (layer F.Cu) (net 12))
 (segment (start 148.891 72.845) (end 148.891 73.345) (width 0.4) (layer F.Cu) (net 9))
 (segment (start 148.081 74.155) (end 146.301 74.155) (width 0.4) (layer F.Cu) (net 9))
 (segment (start 148.081 74.155) (end 148.891 73.345) (width 0.4) (layer F.Cu) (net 9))
 (segment (start 152.791 70.495) (end 152.791 71.945) (width 0.5) (layer B.Cu) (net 9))
 (segment (start 153.301 69.985) (end 152.791 70.495) (width 0.5) (layer B.Cu) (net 9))
 (via (at 153.301 69.985) (size 1) (drill 0.5) (layers F.Cu B.Cu) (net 9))
 (segment (start 152.901 70.385) (end 153.301 69.985) (width 0.5) (layer F.Cu) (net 9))
 (segment (start 152.901 71.295) (end 152.901 70.385) (width 0.5) (layer F.Cu) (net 9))
 (segment (start 152.291 71.905) (end 152.901 71.295) (width 0.5) (layer F.Cu) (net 9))
 (segment (start 149.641 71.905) (end 152.291 71.905) (width 0.5) (layer F.Cu) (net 9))
 (segment (start 148.891 72.655) (end 149.641 71.905) (width 0.5) (layer F.Cu) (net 9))
 (segment (start 155.331 71.945) (end 155.331 72.735) (width 0.5) (layer B.Cu) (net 6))
 (segment (start 155.331 72.735) (end 154.391 73.675) (width 0.5) (layer B.Cu) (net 6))
 (segment (start 154.391 73.675) (end 151.751 73.675) (width 0.5) (layer B.Cu) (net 6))
 (segment (start 151.751 73.675) (end 149.336 76.09) (width 0.5) (layer B.Cu) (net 6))
 (segment (start 149.336 76.09) (end 149.336 81.28) (width 0.5) (layer B.Cu) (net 6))
 (segment (start 149.336 81.28) (end 148.711 81.905) (width 0.5) (layer B.Cu) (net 6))
 (segment (start 148.711 81.905) (end 147.011 81.905) (width 0.5) (layer B.Cu) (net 6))
 (segment (start 147.011 81.905) (end 146.421 81.315) (width 0.5) (layer B.Cu) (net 6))
 (segment (start 146.421 81.315) (end 146.421 78.105) (width 0.5) (layer B.Cu) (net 6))
 (segment (start 146.421 69.405) (end 146.076 69.75) (width 0.5) (layer F.Cu) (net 6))
 (via (at 146.421 69.405) (size 0.6) (drill 0.4) (layers F.Cu B.Cu) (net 6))
 (segment (start 146.421 78.105) (end 146.421 69.405) (width 0.5) (layer B.Cu) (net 6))
 (segment (start 146.341 70.925) (end 146.341 70.015) (width 0.5) (layer F.Cu) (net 6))
 (segment (start 146.341 70.015) (end 146.076 69.75) (width 0.5) (layer F.Cu) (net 6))
 (segment (start 146.301 73.505) (end 146.301 70.965) (width 0.4) (layer F.Cu) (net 6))
 (segment (start 146.301 70.965) (end 146.341 70.925) (width 0.4) (layer F.Cu) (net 6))
 (segment (start 146.076 69.77) (end 146.076 69.75) (width 0.5) (layer F.Cu) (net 6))
 (segment (start 145.061 68.755) (end 146.076 69.77) (width 0.5) (layer F.Cu) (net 6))
 (segment (start 145.061 67.845) (end 145.061 68.755) (width 0.5) (layer F.Cu) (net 6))
 (segment (start 153.021 72.835) (end 154.391 71.465) (width 0.5) (layer F.Cu) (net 3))
 (segment (start 154.391 71.465) (end 154.391 69.555) (width 0.5) (layer F.Cu) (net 3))
 (segment (start 152.681 67.845) (end 154.391 69.555) (width 0.5) (layer F.Cu) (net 3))
 (segment (start 150.991 76.235) (end 153.021 74.205) (width 0.5) (layer F.Cu) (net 3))
 (segment (start 153.021 74.205) (end 153.021 72.835) (width 0.5) (layer F.Cu) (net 3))
 (segment (start 150.991 76.235) (end 150.991 77.225) (width 0.5) (layer F.Cu) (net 3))
 (segment (start 152.516 68.01) (end 152.681 67.845) (width 0.5) (layer F.Cu) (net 3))
 (segment (start 151.471 70.955) (end 151.471 69.585) (width 0.5) (layer F.Cu) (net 4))
 (segment (start 151.471 69.585) (end 150.141 68.255) (width 0.5) (layer F.Cu) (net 4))
 (segment (start 150.141 67.845) (end 150.141 68.255) (width 0.5) (layer F.Cu) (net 4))
 (segment (start 148.891 70.945) (end 148.891 69.665) (width 0.5) (layer F.Cu) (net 5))
 (segment (start 148.891 69.665) (end 147.601 68.375) (width 0.5) (layer F.Cu) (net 5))
 (segment (start 147.601 67.845) (end 147.601 68.375) (width 0.5) (layer F.Cu) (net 5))
 (segment (start 153.191 78.885) (end 153.191 81.245) (width 0.5) (layer F.Cu) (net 39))
 (segment (start 154.311 81.245) (end 153.191 81.245) (width 0.5) (layer F.Cu) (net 39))
 (segment (start 153.191 81.245) (end 151.791 81.245) (width 0.5) (layer F.Cu) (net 39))
 (segment (start 155.391 75.215) (end 155.391 76.595) (width 0.75) (layer F.Cu) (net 40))
 (segment (start 155.391 76.985) (end 155.391 76.595) (width 0.5) (layer F.Cu) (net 40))
 (segment (start 155.391 75.215) (end 156.031 74.575) (width 0.75) (layer F.Cu) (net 40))
 (segment (start 156.031 74.575) (end 156.831 74.575) (width 0.75) (layer F.Cu) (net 40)))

